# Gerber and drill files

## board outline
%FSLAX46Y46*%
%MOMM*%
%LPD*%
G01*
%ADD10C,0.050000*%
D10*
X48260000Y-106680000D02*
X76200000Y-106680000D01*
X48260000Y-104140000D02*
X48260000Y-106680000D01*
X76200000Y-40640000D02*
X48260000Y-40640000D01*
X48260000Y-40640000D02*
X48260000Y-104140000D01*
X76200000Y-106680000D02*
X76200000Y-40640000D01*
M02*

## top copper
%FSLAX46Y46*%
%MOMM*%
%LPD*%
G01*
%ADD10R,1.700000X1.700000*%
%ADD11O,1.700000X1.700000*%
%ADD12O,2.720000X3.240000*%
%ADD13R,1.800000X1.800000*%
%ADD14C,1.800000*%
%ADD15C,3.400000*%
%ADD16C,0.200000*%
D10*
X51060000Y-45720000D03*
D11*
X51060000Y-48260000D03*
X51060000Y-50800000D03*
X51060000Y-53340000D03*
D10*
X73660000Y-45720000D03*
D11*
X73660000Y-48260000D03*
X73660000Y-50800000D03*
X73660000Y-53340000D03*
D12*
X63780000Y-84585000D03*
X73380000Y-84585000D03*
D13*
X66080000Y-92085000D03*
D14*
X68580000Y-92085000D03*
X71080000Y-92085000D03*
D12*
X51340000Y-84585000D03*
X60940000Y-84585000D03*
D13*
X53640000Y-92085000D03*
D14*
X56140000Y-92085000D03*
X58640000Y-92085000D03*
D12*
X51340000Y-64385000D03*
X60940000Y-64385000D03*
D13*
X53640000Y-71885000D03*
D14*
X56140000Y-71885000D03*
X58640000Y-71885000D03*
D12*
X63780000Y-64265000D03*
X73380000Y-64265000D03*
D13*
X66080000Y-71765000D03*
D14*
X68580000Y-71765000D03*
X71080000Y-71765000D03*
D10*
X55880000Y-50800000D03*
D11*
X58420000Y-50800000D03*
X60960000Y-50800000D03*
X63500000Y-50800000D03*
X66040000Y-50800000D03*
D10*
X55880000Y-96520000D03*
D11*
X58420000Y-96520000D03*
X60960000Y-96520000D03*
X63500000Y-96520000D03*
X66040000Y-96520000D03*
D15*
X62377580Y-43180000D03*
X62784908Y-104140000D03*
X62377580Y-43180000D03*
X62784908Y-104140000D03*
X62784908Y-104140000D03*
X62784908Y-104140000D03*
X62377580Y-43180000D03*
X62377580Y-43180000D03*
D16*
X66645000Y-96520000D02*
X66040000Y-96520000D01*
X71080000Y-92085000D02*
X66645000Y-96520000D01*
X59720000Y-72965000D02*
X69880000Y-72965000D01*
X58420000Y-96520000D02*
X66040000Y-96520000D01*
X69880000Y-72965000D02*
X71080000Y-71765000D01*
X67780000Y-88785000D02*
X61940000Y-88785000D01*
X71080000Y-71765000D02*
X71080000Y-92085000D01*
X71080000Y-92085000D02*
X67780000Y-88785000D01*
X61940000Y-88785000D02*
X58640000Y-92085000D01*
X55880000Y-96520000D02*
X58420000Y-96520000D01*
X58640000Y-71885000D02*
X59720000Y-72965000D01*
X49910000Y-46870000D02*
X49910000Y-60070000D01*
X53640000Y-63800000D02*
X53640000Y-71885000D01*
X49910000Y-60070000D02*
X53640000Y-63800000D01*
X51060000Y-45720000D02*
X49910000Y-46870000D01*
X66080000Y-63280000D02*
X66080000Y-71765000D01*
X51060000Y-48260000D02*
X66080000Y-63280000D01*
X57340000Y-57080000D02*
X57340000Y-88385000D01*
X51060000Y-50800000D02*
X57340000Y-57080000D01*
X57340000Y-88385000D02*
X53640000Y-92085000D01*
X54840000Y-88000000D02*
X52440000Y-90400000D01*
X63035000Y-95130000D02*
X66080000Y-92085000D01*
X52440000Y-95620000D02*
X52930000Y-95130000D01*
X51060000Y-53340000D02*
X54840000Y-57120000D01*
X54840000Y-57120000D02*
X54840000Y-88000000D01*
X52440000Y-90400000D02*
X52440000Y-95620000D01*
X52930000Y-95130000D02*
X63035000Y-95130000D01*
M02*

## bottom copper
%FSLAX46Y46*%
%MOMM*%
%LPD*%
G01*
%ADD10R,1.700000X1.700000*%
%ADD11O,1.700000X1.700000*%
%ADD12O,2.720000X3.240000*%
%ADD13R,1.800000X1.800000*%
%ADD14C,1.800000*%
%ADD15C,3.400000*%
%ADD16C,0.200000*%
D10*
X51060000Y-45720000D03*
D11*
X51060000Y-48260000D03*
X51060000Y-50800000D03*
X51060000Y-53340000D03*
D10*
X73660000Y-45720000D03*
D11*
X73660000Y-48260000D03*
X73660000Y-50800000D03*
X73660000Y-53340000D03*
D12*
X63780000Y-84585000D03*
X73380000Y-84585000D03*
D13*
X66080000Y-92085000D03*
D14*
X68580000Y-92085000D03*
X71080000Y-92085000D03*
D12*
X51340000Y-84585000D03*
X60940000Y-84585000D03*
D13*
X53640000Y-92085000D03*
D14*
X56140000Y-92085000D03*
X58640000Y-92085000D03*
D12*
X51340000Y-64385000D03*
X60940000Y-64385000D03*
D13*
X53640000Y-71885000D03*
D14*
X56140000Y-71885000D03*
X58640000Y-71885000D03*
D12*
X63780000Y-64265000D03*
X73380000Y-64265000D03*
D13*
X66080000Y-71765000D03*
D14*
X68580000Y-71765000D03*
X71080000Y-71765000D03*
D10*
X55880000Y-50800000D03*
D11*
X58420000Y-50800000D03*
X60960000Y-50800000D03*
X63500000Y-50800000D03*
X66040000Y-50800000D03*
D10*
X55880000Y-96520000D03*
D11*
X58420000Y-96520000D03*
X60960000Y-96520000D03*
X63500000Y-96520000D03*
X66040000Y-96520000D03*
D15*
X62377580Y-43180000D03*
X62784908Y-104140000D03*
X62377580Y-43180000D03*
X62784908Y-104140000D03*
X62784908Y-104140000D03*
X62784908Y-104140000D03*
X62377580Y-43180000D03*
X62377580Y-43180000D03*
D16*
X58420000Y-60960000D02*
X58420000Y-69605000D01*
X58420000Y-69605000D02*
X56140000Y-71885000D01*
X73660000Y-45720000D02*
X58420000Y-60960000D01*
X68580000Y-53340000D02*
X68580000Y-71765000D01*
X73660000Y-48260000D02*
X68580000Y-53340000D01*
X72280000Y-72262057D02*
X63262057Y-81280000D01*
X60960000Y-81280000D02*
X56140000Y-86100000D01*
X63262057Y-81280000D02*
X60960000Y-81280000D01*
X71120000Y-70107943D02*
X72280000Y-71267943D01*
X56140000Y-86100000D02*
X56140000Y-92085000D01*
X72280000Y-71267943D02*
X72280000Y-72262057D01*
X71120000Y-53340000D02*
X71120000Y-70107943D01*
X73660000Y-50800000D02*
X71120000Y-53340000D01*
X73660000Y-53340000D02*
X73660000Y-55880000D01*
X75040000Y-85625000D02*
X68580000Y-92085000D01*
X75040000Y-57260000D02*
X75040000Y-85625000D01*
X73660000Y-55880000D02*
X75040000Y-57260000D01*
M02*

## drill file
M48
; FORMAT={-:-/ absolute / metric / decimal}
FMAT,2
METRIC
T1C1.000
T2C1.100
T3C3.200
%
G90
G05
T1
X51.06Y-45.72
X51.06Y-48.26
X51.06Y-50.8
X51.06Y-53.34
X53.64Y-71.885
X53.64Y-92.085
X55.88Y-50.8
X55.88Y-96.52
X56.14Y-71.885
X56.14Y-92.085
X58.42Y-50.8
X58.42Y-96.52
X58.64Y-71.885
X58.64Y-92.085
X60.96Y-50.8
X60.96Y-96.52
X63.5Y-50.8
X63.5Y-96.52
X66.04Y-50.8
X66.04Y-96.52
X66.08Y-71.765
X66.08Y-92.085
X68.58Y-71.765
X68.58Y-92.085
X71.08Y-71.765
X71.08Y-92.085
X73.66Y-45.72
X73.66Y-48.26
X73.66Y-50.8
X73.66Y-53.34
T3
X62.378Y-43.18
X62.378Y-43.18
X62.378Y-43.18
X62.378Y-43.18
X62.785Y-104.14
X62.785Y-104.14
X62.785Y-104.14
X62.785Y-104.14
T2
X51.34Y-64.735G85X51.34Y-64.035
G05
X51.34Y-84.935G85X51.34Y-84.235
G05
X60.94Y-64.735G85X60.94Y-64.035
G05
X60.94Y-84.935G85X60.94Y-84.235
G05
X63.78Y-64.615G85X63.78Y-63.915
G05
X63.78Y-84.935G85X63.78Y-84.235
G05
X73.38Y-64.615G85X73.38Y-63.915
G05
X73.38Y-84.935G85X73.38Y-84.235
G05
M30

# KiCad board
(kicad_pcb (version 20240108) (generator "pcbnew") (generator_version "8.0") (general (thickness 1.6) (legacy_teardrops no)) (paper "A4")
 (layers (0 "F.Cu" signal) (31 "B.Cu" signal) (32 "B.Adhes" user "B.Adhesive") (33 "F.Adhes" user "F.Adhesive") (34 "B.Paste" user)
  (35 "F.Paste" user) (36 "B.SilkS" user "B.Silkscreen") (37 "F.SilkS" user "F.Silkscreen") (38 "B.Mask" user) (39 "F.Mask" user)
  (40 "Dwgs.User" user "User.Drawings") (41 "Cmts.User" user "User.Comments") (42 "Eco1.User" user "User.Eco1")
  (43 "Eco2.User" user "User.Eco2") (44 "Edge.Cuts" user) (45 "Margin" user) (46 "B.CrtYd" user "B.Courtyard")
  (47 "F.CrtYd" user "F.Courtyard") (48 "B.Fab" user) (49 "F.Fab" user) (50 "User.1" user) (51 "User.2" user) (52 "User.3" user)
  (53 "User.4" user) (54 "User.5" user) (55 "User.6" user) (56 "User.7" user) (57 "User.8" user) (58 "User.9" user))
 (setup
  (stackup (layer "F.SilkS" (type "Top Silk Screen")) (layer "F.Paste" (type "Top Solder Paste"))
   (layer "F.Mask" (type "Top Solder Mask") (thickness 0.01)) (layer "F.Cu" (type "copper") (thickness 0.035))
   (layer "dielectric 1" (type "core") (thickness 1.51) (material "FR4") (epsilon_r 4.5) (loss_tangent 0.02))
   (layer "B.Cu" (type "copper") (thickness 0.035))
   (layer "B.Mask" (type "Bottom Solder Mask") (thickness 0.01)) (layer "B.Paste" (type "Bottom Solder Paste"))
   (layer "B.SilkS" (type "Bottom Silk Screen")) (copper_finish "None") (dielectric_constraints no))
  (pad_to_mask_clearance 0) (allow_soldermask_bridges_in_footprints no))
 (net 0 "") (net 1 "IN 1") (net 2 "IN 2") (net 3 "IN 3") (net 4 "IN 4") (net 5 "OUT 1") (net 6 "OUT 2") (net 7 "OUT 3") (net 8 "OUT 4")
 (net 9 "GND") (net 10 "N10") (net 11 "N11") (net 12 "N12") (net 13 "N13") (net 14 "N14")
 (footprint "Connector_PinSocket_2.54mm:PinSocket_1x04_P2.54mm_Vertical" (layer "F.Cu") (at 51.06 45.72)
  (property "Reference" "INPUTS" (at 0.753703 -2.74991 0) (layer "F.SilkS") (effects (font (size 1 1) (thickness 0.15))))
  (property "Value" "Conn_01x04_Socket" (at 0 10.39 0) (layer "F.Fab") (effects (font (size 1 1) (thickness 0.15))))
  (pad "1" thru_hole rect (at 0 0) (size 1.7 1.7) (drill 1) (layers "*.Cu" "*.Mask") (remove_unused_layers no) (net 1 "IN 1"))
  (pad "2" thru_hole oval (at 0 2.54) (size 1.7 1.7) (drill 1) (layers "*.Cu" "*.Mask") (remove_unused_layers no) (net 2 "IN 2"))
  (pad "3" thru_hole oval (at 0 5.08) (size 1.7 1.7) (drill 1) (layers "*.Cu" "*.Mask") (remove_unused_layers no) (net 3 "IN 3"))
  (pad "4" thru_hole oval (at 0 7.62) (size 1.7 1.7) (drill 1) (layers "*.Cu" "*.Mask") (remove_unused_layers no) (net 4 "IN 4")))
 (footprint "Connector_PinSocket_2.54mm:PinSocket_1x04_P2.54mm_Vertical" (layer "F.Cu") (at 73.66 45.72)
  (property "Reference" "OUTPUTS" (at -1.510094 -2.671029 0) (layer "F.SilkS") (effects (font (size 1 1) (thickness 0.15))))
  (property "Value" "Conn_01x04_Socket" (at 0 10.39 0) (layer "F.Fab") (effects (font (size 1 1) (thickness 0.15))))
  (pad "1" thru_hole rect (at 0 0) (size 1.7 1.7) (drill 1) (layers "*.Cu" "*.Mask") (remove_unused_layers no) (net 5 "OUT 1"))
  (pad "2" thru_hole oval (at 0 2.54) (size 1.7 1.7) (drill 1) (layers "*.Cu" "*.Mask") (remove_unused_layers no) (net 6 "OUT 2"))
  (pad "3" thru_hole oval (at 0 5.08) (size 1.7 1.7) (drill 1) (layers "*.Cu" "*.Mask") (remove_unused_layers no) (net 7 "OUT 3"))
  (pad "4" thru_hole oval (at 0 7.62) (size 1.7 1.7) (drill 1) (layers "*.Cu" "*.Mask") (remove_unused_layers no) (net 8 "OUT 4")))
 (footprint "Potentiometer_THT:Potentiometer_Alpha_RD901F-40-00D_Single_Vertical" (layer "F.Cu") (at 66.08 92.085 90)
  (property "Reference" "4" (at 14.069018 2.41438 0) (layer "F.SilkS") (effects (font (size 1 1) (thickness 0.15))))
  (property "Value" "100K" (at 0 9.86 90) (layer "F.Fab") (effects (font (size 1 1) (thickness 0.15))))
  (pad "" thru_hole oval (at 7.5 -2.3 180) (size 2.72 3.24) (drill oval 1.1 1.8) (layers "*.Cu" "*.Mask") (remove_unused_layers no))
  (pad "" thru_hole oval (at 7.5 7.3 180) (size 2.72 3.24) (drill oval 1.1 1.8) (layers "*.Cu" "*.Mask") (remove_unused_layers no))
  (pad "1" thru_hole rect (at 0 0 180) (size 1.8 1.8) (drill 1) (layers "*.Cu" "*.Mask") (remove_unused_layers no) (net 4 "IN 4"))
  (pad "2" thru_hole circle (at 0 2.5 180) (size 1.8 1.8) (drill 1) (layers "*.Cu" "*.Mask") (remove_unused_layers no) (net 8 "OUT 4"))
  (pad "3" thru_hole circle (at 0 5 180) (size 1.8 1.8) (drill 1) (layers "*.Cu" "*.Mask") (remove_unused_layers no) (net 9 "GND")))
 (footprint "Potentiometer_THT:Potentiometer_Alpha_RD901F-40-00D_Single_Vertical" (layer "F.Cu") (at 53.64 92.085 90)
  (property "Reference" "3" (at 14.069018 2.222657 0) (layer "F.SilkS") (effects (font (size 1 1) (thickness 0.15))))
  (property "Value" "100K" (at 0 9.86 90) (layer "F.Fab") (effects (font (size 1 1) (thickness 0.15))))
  (pad "" thru_hole oval (at 7.5 -2.3 180) (size 2.72 3.24) (drill oval 1.1 1.8) (layers "*.Cu" "*.Mask") (remove_unused_layers no))
  (pad "" thru_hole oval (at 7.5 7.3 180) (size 2.72 3.24) (drill oval 1.1 1.8) (layers "*.Cu" "*.Mask") (remove_unused_layers no))
  (pad "1" thru_hole rect (at 0 0 180) (size 1.8 1.8) (drill 1) (layers "*.Cu" "*.Mask") (remove_unused_layers no) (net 3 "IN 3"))
  (pad "2" thru_hole circle (at 0 2.5 180) (size 1.8 1.8) (drill 1) (layers "*.Cu" "*.Mask") (remove_unused_layers no) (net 7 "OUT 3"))
  (pad "3" thru_hole circle (at 0 5 180) (size 1.8 1.8) (drill 1) (layers "*.Cu" "*.Mask") (remove_unused_layers no) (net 9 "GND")))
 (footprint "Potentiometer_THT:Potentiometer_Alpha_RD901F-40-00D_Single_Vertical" (layer "F.Cu") (at 53.64 71.885 90)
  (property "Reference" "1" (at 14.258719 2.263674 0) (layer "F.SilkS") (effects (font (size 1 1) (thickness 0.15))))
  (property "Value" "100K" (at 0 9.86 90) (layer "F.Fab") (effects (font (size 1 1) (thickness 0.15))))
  (pad "" thru_hole oval (at 7.5 -2.3 180) (size 2.72 3.24) (drill oval 1.1 1.8) (layers "*.Cu" "*.Mask") (remove_unused_layers no))
  (pad "" thru_hole oval (at 7.5 7.3 180) (size 2.72 3.24) (drill oval 1.1 1.8) (layers "*.Cu" "*.Mask") (remove_unused_layers no))
  (pad "1" thru_hole rect (at 0 0 180) (size 1.8 1.8) (drill 1) (layers "*.Cu" "*.Mask") (remove_unused_layers no) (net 1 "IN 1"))
  (pad "2" thru_hole circle (at 0 2.5 180) (size 1.8 1.8) (drill 1) (layers "*.Cu" "*.Mask") (remove_unused_layers no) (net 5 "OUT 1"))
  (pad "3" thru_hole circle (at 0 5 180) (size 1.8 1.8) (drill 1) (layers "*.Cu" "*.Mask") (remove_unused_layers no) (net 9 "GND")))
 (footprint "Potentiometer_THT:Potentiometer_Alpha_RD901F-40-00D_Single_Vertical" (layer "F.Cu") (at 66.08 71.765 90)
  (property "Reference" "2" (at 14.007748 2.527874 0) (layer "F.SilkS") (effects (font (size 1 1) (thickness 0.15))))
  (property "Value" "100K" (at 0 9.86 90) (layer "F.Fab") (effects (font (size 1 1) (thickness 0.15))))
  (pad "" thru_hole oval (at 7.5 -2.3 180) (size 2.72 3.24) (drill oval 1.1 1.8) (layers "*.Cu" "*.Mask") (remove_unused_layers no))
  (pad "" thru_hole oval (at 7.5 7.3 180) (size 2.72 3.24) (drill oval 1.1 1.8) (layers "*.Cu" "*.Mask") (remove_unused_layers no))
  (pad "1" thru_hole rect (at 0 0 180) (size 1.8 1.8) (drill 1) (layers "*.Cu" "*.Mask") (remove_unused_layers no) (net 2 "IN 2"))
  (pad "2" thru_hole circle (at 0 2.5 180) (size 1.8 1.8) (drill 1) (layers "*.Cu" "*.Mask") (remove_unused_layers no) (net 6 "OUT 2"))
  (pad "3" thru_hole circle (at 0 5 180) (size 1.8 1.8) (drill 1) (layers "*.Cu" "*.Mask") (remove_unused_layers no) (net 9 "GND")))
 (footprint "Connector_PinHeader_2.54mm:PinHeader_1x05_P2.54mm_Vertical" (layer "B.Cu") (at 55.88 50.8 -90)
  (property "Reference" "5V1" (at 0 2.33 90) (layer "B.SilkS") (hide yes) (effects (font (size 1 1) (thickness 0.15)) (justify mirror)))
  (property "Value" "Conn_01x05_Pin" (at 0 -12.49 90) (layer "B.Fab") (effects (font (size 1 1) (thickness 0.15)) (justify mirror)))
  (pad "1" thru_hole rect (at 0 0 270) (size 1.7 1.7) (drill 1) (layers "*.Cu" "*.Mask") (remove_unused_layers no) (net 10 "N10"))
  (pad "2" thru_hole oval (at 0 -2.54 270) (size 1.7 1.7) (drill 1) (layers "*.Cu" "*.Mask") (remove_unused_layers no) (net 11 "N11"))
  (pad "3" thru_hole oval (at 0 -5.08 270) (size 1.7 1.7) (drill 1) (layers "*.Cu" "*.Mask") (remove_unused_layers no) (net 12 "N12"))
  (pad "4" thru_hole oval (at 0 -7.62 270) (size 1.7 1.7) (drill 1) (layers "*.Cu" "*.Mask") (remove_unused_layers no) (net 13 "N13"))
  (pad "5" thru_hole oval (at 0 -10.16 270) (size 1.7 1.7) (drill 1) (layers "*.Cu" "*.Mask") (remove_unused_layers no) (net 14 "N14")))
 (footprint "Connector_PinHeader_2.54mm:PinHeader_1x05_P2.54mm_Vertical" (layer "B.Cu") (at 55.88 96.52 -90)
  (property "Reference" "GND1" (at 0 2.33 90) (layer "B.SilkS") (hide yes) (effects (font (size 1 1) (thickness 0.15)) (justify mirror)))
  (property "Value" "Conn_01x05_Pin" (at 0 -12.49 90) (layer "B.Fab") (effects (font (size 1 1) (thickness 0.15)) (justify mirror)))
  (pad "1" thru_hole rect (at 0 0 270) (size 1.7 1.7) (drill 1) (layers "*.Cu" "*.Mask") (remove_unused_layers no) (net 9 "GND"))
  (pad "2" thru_hole oval (at 0 -2.54 270) (size 1.7 1.7) (drill 1) (layers "*.Cu" "*.Mask") (remove_unused_layers no) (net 9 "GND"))
  (pad "3" thru_hole oval (at 0 -5.08 270) (size 1.7 1.7) (drill 1) (layers "*.Cu" "*.Mask") (remove_unused_layers no) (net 9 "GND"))
  (pad "4" thru_hole oval (at 0 -7.62 270) (size 1.7 1.7) (drill 1) (layers "*.Cu" "*.Mask") (remove_unused_layers no) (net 9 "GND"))
  (pad "5" thru_hole oval (at 0 -10.16 270) (size 1.7 1.7) (drill 1) (layers "*.Cu" "*.Mask") (remove_unused_layers no) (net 9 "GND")))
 (gr_line (start 48.26 106.68) (end 76.2 106.68) (stroke (width 0.05) (type default)) (layer "Edge.Cuts"))
 (gr_line (start 48.26 104.14) (end 48.26 106.68) (stroke (width 0.05) (type default)) (layer "Edge.Cuts"))
 (gr_line (start 76.2 40.64) (end 48.26 40.64) (stroke (width 0.05) (type default)) (layer "Edge.Cuts"))
 (gr_line (start 48.26 40.64) (end 48.26 104.14) (stroke (width 0.05) (type default)) (layer "Edge.Cuts"))
 (gr_line (start 76.2 106.68) (end 76.2 40.64) (stroke (width 0.05) (type default)) (layer "Edge.Cuts"))
 (via (at 62.37758 43.18) (size 3.4) (drill 3.2) (layers "F.Cu" "B.Cu") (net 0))
 (via (at 62.784908 104.14) (size 3.4) (drill 3.2) (layers "F.Cu" "B.Cu") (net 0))
 (via (at 62.37758 43.18) (size 3.4) (drill 3.2) (layers "F.Cu" "B.Cu") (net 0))
 (via (at 62.784908 104.14) (size 3.4) (drill 3.2) (layers "F.Cu" "B.Cu") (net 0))
 (via (at 62.784908 104.14) (size 3.4) (drill 3.2) (layers "F.Cu" "B.Cu") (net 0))
 (via (at 62.784908 104.14) (size 3.4) (drill 3.2) (layers "F.Cu" "B.Cu") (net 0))
 (via (at 62.37758 43.18) (size 3.4) (drill 3.2) (layers "F.Cu" "B.Cu") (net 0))
 (via (at 62.37758 43.18) (size 3.4) (drill 3.2) (layers "F.Cu" "B.Cu") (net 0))
 (segment (start 66.645 96.52) (end 66.04 96.52) (width 0.2) (layer "F.Cu") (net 9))
 (segment (start 71.08 92.085) (end 66.645 96.52) (width 0.2) (layer "F.Cu") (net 9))
 (segment (start 59.72 72.965) (end 69.88 72.965) (width 0.2) (layer "F.Cu") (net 9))
 (segment (start 58.42 96.52) (end 66.04 96.52) (width 0.2) (layer "F.Cu") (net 9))
 (segment (start 69.88 72.965) (end 71.08 71.765) (width 0.2) (layer "F.Cu") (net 9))
 (segment (start 67.78 88.785) (end 61.94 88.785) (width 0.2) (layer "F.Cu") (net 9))
 (segment (start 71.08 71.765) (end 71.08 92.085) (width 0.2) (layer "F.Cu") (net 9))
 (segment (start 71.08 92.085) (end 67.78 88.785) (width 0.2) (layer "F.Cu") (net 9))
 (segment (start 61.94 88.785) (end 58.64 92.085) (width 0.2) (layer "F.Cu") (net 9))
 (segment (start 55.88 96.52) (end 58.42 96.52) (width 0.2) (layer "F.Cu") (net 9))
 (segment (start 58.64 71.885) (end 59.72 72.965) (width 0.2) (layer "F.Cu") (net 9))
 (segment (start 58.42 60.96) (end 58.42 69.605) (width 0.2) (layer "B.Cu") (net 5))
 (segment (start 58.42 69.605) (end 56.14 71.885) (width 0.2) (layer "B.Cu") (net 5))
 (segment (start 73.66 45.72) (end 58.42 60.96) (width 0.2) (layer "B.Cu") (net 5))
 (segment (start 49.91 46.87) (end 49.91 60.07) (width 0.2) (layer "F.Cu") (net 1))
 (segment (start 53.64 63.8) (end 53.64 71.885) (width 0.2) (layer "F.Cu") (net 1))
 (segment (start 49.91 60.07) (end 53.64 63.8) (width 0.2) (layer "F.Cu") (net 1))
 (segment (start 51.06 45.72) (end 49.91 46.87) (width 0.2) (layer "F.Cu") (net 1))
 (segment (start 68.58 53.34) (end 68.58 71.765) (width 0.2) (layer "B.Cu") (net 6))
 (segment (start 73.66 48.26) (end 68.58 53.34) (width 0.2) (layer "B.Cu") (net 6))
 (segment (start 66.08 63.28) (end 66.08 71.765) (width 0.2) (layer "F.Cu") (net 2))
 (segment (start 51.06 48.26) (end 66.08 63.28) (width 0.2) (layer "F.Cu") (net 2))
 (segment (start 57.34 57.08) (end 57.34 88.385) (width 0.2) (layer "F.Cu") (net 3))
 (segment (start 51.06 50.8) (end 57.34 57.08) (width 0.2) (layer "F.Cu") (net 3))
 (segment (start 57.34 88.385) (end 53.64 92.085) (width 0.2) (layer "F.Cu") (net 3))
 (segment (start 72.28 72.262057) (end 63.262057 81.28) (width 0.2) (layer "B.Cu") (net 7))
 (segment (start 60.96 81.28) (end 56.14 86.1) (width 0.2) (layer "B.Cu") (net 7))
 (segment (start 63.262057 81.28) (end 60.96 81.28) (width 0.2) (layer "B.Cu") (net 7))
 (segment (start 71.12 70.107943) (end 72.28 71.267943) (width 0.2) (layer "B.Cu") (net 7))
 (segment (start 56.14 86.1) (end 56.14 92.085) (width 0.2) (layer "B.Cu") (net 7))
 (segment (start 72.28 71.267943) (end 72.28 72.262057) (width 0.2) (layer "B.Cu") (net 7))
 (segment (start 71.12 53.34) (end 71.12 70.107943) (width 0.2) (layer "B.Cu") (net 7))
 (segment (start 73.66 50.8) (end 71.12 53.34) (width 0.2) (layer "B.Cu") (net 7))
 (segment (start 54.84 88) (end 52.44 90.4) (width 0.2) (layer "F.Cu") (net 4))
 (segment (start 63.035 95.13) (end 66.08 92.085) (width 0.2) (layer "F.Cu") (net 4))
 (segment (start 52.44 95.62) (end 52.93 95.13) (width 0.2) (layer "F.Cu") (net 4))
 (segment (start 51.06 53.34) (end 54.84 57.12) (width 0.2) (layer "F.Cu") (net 4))
 (segment (start 54.84 57.12) (end 54.84 88) (width 0.2) (layer "F.Cu") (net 4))
 (segment (start 52.44 90.4) (end 52.44 95.62) (width 0.2) (layer "F.Cu") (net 4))
 (segment (start 52.93 95.13) (end 63.035 95.13) (width 0.2) (layer "F.Cu") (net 4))
 (segment (start 73.66 53.34) (end 73.66 55.88) (width 0.2) (layer "B.Cu") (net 8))
 (segment (start 75.04 85.625) (end 68.58 92.085) (width 0.2) (layer "B.Cu") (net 8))
 (segment (start 75.04 57.26) (end 75.04 85.625) (width 0.2) (layer "B.Cu") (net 8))
 (segment (start 73.66 55.88) (end 75.04 57.26) (width 0.2) (layer "B.Cu") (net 8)))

